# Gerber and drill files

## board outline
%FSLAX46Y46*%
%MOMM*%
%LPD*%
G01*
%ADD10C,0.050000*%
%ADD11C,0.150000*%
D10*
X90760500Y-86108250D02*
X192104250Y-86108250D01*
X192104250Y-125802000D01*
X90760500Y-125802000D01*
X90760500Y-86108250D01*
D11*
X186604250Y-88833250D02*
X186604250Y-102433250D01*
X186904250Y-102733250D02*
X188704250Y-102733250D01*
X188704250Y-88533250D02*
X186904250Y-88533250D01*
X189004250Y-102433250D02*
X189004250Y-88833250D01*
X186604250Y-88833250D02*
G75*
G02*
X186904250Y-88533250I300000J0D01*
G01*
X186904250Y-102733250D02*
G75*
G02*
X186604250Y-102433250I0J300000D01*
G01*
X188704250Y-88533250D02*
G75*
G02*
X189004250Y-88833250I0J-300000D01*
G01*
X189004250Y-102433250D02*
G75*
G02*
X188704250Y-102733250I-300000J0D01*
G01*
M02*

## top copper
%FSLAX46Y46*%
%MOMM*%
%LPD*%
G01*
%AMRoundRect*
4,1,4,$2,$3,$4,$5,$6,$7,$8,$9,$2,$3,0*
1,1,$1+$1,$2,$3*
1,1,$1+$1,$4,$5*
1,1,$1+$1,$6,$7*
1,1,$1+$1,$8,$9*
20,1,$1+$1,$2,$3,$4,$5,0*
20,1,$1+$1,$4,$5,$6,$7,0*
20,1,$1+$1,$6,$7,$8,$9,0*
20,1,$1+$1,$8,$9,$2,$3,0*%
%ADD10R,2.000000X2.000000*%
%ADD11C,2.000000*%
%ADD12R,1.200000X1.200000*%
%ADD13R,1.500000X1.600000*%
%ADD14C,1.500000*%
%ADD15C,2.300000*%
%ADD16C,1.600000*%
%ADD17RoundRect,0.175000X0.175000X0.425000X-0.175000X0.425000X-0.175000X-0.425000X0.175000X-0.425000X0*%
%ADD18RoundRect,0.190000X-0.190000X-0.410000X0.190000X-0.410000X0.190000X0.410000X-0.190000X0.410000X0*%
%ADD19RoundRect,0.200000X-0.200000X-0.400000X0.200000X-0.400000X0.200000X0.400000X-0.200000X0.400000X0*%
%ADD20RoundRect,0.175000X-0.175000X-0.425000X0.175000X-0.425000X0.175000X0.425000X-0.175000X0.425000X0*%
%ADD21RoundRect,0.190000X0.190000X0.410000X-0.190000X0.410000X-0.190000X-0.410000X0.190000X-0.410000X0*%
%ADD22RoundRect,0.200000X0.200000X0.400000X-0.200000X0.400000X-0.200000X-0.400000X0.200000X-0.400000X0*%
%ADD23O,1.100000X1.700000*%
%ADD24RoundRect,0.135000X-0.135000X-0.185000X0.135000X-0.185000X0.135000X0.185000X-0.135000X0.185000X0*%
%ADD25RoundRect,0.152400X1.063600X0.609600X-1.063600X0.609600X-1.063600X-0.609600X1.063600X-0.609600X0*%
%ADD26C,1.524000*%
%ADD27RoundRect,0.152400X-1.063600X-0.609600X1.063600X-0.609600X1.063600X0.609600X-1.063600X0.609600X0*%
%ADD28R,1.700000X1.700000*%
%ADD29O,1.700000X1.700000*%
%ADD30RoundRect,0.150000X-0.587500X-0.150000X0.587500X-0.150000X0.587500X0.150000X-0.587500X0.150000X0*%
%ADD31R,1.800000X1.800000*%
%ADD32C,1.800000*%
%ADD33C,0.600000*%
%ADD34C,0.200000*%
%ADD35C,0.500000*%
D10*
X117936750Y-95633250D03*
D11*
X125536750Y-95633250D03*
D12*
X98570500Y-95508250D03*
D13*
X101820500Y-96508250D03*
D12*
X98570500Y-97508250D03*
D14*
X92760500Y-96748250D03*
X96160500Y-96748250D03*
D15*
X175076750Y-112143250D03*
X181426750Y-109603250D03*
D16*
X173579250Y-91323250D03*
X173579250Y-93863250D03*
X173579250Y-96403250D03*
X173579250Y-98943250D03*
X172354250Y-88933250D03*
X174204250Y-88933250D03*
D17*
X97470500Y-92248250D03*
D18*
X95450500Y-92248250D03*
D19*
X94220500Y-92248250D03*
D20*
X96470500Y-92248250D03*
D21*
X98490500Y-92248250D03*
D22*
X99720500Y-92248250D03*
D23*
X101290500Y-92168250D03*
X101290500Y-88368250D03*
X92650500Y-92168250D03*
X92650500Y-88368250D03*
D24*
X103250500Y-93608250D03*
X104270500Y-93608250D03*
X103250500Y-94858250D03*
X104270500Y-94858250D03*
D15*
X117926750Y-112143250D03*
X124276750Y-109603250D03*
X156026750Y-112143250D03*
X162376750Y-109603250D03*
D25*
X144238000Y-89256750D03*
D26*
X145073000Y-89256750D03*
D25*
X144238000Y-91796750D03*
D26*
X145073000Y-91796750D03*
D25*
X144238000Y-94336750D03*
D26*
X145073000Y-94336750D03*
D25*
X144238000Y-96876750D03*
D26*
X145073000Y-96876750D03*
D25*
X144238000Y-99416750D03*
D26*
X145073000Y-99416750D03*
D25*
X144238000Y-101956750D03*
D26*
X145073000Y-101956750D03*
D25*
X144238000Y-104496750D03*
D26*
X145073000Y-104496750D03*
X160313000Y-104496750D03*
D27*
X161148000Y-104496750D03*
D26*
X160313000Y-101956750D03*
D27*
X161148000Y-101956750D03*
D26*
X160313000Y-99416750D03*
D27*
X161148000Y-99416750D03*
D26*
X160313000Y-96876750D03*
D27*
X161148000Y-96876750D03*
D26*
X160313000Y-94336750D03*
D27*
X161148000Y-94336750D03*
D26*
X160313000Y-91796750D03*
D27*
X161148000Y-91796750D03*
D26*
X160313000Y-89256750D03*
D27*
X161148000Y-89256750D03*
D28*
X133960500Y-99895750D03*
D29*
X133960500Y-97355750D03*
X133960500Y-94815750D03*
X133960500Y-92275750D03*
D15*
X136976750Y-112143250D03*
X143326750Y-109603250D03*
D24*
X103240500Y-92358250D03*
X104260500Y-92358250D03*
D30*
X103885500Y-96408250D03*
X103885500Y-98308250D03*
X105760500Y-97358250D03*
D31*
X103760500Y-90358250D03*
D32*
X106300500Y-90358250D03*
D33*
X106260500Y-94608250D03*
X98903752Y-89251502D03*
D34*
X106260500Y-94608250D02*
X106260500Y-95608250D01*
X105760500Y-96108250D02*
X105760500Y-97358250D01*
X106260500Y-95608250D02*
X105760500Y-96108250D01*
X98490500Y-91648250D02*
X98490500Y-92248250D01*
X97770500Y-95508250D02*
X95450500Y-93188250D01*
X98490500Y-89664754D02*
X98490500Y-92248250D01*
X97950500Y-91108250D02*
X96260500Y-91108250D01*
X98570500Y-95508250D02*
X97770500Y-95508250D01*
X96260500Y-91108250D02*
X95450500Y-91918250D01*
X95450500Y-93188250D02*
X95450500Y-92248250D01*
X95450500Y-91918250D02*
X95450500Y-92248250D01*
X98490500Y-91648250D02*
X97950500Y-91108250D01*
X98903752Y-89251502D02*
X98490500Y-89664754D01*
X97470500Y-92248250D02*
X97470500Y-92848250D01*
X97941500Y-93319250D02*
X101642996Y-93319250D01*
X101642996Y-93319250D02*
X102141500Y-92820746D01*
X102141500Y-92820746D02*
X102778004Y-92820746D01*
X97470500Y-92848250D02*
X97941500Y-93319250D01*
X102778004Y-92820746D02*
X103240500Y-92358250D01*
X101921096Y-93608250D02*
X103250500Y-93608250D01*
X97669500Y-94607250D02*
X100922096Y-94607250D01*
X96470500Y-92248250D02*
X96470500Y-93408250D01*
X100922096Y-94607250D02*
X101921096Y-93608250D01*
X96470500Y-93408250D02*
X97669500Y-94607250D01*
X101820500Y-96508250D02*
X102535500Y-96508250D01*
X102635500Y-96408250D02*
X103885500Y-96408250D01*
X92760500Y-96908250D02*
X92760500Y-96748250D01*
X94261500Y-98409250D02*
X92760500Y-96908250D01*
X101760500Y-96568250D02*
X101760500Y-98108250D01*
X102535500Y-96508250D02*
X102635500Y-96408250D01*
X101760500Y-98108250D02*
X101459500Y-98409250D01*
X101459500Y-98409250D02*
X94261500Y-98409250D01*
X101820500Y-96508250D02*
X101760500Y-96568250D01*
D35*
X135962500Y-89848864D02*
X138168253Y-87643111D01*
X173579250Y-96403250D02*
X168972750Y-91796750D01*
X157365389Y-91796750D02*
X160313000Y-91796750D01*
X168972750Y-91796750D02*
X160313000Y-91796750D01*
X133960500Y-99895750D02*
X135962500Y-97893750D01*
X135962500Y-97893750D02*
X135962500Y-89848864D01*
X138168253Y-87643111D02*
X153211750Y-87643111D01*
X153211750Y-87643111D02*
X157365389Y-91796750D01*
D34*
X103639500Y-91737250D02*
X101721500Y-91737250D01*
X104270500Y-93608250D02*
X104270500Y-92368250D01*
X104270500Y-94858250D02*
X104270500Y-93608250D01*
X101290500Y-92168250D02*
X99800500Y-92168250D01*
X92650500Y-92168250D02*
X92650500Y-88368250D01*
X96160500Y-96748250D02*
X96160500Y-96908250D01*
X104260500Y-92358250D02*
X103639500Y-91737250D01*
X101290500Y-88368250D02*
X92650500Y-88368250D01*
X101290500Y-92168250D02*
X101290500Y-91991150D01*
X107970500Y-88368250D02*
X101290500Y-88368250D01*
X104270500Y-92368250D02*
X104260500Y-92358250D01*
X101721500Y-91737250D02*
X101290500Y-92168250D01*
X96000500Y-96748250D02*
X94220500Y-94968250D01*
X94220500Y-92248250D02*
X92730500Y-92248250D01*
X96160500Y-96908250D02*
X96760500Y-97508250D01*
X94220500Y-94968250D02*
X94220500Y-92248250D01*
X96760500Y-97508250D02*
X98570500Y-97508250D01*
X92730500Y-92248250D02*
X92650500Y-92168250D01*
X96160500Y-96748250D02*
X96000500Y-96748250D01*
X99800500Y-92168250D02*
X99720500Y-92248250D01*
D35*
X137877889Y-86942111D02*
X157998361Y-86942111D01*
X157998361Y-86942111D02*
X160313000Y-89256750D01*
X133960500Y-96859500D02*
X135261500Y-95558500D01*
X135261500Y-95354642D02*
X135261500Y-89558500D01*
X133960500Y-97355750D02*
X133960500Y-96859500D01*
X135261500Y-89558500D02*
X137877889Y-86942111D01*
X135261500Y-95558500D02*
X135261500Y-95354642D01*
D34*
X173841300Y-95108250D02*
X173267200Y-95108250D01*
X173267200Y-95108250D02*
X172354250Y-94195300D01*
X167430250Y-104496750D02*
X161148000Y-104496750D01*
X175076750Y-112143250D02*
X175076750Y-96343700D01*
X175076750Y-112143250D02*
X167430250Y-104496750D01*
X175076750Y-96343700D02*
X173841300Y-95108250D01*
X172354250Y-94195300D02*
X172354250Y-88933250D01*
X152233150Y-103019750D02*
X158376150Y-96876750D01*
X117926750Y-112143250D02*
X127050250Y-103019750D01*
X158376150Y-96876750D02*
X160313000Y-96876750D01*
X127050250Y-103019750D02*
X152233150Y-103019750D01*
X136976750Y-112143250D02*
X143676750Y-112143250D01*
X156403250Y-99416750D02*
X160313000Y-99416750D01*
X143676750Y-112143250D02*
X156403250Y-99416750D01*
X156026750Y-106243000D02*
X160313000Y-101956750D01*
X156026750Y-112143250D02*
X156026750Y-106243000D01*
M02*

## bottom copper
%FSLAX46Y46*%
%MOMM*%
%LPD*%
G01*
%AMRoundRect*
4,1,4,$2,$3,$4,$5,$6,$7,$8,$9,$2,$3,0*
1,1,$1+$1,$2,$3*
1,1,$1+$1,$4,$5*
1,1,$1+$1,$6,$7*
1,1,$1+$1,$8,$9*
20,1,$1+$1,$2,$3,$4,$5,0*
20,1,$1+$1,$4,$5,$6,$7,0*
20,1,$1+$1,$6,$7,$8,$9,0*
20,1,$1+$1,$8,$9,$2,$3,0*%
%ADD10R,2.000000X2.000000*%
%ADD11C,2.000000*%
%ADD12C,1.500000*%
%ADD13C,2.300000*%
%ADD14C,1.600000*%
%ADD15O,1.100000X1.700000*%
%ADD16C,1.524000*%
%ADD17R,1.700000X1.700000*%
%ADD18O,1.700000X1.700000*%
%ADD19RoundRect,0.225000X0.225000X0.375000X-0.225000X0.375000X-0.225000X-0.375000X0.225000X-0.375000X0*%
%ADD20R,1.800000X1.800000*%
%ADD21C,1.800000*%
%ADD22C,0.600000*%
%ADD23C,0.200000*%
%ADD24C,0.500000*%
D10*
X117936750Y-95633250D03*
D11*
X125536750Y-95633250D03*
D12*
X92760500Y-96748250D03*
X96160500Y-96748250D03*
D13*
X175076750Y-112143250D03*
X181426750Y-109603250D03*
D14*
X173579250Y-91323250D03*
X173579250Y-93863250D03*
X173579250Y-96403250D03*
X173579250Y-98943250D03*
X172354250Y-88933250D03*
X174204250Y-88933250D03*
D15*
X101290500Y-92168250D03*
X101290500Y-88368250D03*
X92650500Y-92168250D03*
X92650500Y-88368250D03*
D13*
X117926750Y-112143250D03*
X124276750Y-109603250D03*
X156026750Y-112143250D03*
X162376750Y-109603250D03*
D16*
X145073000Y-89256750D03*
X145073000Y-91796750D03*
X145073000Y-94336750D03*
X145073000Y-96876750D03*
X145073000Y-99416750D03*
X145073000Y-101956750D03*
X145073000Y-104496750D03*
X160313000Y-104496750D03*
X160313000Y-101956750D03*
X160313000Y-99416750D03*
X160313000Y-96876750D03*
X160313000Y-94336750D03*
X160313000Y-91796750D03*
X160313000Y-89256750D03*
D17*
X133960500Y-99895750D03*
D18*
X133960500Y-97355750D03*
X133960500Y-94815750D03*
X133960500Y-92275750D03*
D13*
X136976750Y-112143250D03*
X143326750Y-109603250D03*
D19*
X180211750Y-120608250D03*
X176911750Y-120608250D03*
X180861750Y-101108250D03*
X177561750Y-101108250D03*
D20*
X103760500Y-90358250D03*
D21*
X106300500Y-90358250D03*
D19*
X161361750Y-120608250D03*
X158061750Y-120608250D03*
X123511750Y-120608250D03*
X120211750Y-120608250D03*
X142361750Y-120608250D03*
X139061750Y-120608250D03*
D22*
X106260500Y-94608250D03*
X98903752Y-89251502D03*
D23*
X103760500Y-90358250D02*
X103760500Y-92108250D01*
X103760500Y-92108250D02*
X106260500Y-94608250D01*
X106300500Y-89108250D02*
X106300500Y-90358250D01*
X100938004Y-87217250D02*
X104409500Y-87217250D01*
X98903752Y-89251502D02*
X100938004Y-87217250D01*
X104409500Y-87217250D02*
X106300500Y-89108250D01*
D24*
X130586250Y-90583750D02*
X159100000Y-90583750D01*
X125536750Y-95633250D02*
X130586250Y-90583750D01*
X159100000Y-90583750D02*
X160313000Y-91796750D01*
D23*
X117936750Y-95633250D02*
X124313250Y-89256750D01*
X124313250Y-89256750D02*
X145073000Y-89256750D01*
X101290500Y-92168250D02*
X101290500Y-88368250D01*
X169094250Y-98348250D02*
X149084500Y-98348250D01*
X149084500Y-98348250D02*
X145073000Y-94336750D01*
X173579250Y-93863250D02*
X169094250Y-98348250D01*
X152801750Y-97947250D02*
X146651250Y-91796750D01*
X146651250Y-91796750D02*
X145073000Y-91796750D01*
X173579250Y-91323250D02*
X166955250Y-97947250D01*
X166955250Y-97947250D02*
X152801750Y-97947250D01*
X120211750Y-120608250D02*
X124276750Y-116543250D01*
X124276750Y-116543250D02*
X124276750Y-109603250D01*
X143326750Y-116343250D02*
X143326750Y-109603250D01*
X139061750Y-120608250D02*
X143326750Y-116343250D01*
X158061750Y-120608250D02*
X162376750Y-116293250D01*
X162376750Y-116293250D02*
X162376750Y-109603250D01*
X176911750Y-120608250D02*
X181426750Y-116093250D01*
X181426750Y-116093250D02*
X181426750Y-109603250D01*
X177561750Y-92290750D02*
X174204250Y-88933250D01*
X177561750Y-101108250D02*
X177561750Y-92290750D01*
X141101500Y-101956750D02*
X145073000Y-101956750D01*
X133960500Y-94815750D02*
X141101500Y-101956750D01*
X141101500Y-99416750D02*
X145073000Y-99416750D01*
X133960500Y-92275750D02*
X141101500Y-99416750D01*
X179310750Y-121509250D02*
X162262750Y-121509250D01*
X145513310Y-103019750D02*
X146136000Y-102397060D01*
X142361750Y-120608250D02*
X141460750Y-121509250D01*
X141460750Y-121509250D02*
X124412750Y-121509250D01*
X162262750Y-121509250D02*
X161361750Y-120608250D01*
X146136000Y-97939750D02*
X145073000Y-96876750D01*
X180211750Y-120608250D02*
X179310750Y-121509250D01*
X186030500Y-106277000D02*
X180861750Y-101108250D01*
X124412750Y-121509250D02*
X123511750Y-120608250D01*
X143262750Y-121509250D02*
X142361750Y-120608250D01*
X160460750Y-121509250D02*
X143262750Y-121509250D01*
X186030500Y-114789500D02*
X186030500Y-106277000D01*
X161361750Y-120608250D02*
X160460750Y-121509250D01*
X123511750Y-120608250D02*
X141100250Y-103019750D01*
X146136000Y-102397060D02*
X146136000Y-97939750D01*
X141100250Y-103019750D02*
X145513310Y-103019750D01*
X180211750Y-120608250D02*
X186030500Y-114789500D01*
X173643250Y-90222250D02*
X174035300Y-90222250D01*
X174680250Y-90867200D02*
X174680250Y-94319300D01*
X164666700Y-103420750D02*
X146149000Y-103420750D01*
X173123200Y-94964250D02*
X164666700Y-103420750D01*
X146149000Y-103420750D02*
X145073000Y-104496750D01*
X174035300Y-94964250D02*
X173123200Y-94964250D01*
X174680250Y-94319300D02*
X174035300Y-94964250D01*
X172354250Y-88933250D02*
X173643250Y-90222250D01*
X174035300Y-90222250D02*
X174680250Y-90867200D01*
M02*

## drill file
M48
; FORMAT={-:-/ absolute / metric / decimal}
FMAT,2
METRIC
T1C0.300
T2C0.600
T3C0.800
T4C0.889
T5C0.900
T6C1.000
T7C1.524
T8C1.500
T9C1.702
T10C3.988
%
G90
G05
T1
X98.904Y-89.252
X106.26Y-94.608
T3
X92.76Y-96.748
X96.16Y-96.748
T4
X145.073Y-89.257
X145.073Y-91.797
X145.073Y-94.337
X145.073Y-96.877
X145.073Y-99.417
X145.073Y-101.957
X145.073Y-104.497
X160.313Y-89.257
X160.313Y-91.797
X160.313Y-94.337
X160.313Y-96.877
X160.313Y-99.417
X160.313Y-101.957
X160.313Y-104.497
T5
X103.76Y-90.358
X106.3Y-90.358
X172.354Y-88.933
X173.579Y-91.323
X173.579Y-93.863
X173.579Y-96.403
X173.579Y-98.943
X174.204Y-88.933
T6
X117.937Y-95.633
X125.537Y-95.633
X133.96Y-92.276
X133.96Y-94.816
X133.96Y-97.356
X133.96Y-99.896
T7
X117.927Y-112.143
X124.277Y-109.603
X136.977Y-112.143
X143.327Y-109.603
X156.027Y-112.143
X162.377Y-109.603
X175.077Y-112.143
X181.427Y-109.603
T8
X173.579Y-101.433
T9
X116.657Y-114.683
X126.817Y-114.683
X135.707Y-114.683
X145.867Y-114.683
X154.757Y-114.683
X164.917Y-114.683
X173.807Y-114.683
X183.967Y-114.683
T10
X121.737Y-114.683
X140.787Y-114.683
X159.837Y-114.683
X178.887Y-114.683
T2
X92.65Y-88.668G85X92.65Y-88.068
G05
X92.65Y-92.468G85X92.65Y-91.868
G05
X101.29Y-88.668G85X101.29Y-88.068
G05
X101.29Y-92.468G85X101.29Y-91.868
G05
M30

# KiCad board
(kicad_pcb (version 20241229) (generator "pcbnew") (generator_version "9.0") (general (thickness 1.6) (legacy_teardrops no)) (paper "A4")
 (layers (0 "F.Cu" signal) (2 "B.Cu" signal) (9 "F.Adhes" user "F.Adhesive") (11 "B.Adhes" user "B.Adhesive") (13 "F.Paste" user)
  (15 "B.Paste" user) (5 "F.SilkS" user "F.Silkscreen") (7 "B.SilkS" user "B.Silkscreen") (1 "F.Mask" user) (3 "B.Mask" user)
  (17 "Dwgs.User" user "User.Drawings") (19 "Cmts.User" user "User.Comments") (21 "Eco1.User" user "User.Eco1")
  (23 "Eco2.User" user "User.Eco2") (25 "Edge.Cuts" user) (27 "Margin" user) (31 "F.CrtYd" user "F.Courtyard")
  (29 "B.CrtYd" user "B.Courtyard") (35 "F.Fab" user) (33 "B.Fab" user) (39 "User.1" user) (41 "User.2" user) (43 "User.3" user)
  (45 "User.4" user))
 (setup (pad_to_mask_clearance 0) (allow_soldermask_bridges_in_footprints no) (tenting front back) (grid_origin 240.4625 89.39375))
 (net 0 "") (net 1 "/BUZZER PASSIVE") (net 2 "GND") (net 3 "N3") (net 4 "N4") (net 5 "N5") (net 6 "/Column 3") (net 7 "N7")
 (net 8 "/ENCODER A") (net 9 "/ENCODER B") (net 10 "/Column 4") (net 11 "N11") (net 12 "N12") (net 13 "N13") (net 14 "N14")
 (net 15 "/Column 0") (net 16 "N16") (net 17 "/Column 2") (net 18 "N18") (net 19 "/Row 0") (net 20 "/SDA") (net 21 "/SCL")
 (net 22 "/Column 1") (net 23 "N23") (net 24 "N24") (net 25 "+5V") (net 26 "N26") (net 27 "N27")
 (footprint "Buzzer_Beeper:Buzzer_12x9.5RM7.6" (layer "F.Cu") (at 117.93675 95.63325)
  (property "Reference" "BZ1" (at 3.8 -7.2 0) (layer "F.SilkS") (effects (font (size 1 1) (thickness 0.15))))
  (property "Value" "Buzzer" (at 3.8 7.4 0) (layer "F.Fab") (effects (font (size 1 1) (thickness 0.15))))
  (pad "1" thru_hole rect (at 0 0) (size 2 2) (drill 1) (layers "*.Cu" "*.Mask") (remove_unused_layers no) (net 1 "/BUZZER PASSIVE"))
  (pad "2" thru_hole circle (at 7.6 0) (size 2 2) (drill 1) (layers "*.Cu" "*.Mask") (remove_unused_layers no) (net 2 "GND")))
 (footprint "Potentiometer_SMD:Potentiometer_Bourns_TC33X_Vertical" (layer "F.Cu") (at 100.3705 96.50825)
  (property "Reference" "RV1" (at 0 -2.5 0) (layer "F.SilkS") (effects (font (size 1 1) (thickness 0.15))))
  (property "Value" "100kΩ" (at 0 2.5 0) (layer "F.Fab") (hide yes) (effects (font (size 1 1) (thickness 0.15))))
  (pad "1" smd rect (at -1.8 -1) (size 1.2 1.2) (layers "F.Cu" "F.Mask" "F.Paste") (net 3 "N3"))
  (pad "2" smd rect (at 1.45 0) (size 1.5 1.6) (layers "F.Cu" "F.Mask" "F.Paste") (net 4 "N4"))
  (pad "3" smd rect (at -1.8 1) (size 1.2 1.2) (layers "F.Cu" "F.Mask" "F.Paste") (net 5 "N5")))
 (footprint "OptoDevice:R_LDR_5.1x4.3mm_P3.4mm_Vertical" (layer "F.Cu") (at 92.7605 96.74825)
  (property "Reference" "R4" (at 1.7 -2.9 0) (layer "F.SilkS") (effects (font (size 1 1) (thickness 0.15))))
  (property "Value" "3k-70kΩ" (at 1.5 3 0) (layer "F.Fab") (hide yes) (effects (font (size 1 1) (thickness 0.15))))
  (pad "1" thru_hole circle (at 0 0) (size 1.5 1.5) (drill 0.8) (layers "*.Cu" "*.Mask") (remove_unused_layers no) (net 4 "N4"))
  (pad "2" thru_hole circle (at 3.4 0) (size 1.5 1.5) (drill 0.8) (layers "*.Cu" "*.Mask") (remove_unused_layers no) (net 5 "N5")))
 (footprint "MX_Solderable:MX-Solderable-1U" (layer "F.Cu") (at 178.88675 114.68325)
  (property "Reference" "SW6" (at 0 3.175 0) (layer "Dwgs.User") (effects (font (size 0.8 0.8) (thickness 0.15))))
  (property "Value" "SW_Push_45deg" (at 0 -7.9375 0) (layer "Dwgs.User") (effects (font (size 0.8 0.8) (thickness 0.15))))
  (pad "" np_thru_hole circle (at -5.08 0 48.099) (size 1.7018 1.7018) (drill 1.7018) (layers "*.Cu" "*.Mask"))
  (pad "" np_thru_hole circle (at 0 0) (size 3.9878 3.9878) (drill 3.9878) (layers "*.Cu" "*.Mask"))
  (pad "" np_thru_hole circle (at 5.08 0 48.099) (size 1.7018 1.7018) (drill 1.7018) (layers "*.Cu" "*.Mask"))
  (pad "1" thru_hole circle (at -3.81 -2.54) (size 2.3 2.3) (drill 1.524) (layers "*.Cu" "B.Mask") (remove_unused_layers no)
   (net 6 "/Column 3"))
  (pad "2" thru_hole circle (at 2.54 -5.08) (size 2.3 2.3) (drill 1.524) (layers "*.Cu" "B.Mask") (remove_unused_layers no) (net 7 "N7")))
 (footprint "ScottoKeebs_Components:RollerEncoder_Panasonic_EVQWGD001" (layer "F.Cu") (at 179.20425 95.13325)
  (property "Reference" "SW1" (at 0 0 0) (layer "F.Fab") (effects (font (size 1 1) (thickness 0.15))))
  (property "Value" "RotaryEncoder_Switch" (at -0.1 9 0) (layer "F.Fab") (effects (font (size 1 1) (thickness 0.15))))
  (fp_line (start 7.4 -6.3) (end 7.4 7.3) (stroke (width 0.15) (type solid)) (layer "Edge.Cuts"))
  (fp_line (start 7.7 7.6) (end 9.5 7.6) (stroke (width 0.15) (type solid)) (layer "Edge.Cuts"))
  (fp_line (start 9.5 -6.6) (end 7.7 -6.6) (stroke (width 0.15) (type solid)) (layer "Edge.Cuts"))
  (fp_line (start 9.8 7.3) (end 9.8 -6.3) (stroke (width 0.15) (type solid)) (layer "Edge.Cuts"))
  (fp_arc (start 7.4 -6.3) (mid 7.487868 -6.512132) (end 7.7 -6.6) (stroke (width 0.15) (type solid)) (layer "Edge.Cuts"))
  (fp_arc (start 7.7 7.6) (mid 7.487868 7.512132) (end 7.4 7.3) (stroke (width 0.15) (type solid)) (layer "Edge.Cuts"))
  (fp_arc (start 9.5 -6.6) (mid 9.712132 -6.512132) (end 9.8 -6.3) (stroke (width 0.15) (type solid)) (layer "Edge.Cuts"))
  (fp_arc (start 9.8 7.3) (mid 9.712132 7.512132) (end 9.5 7.6) (stroke (width 0.15) (type solid)) (layer "Edge.Cuts"))
  (pad "" np_thru_hole circle (at -5.625 6.3) (size 1.5 1.5) (drill 1.5) (layers "*.Cu" "*.Mask"))
  (pad "A" thru_hole circle (at -5.625 -3.81) (size 1.6 1.6) (drill 0.9) (layers "*.Cu" "*.Mask") (remove_unused_layers no)
   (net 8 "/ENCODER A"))
  (pad "B" thru_hole circle (at -5.625 -1.27) (size 1.6 1.6) (drill 0.9) (layers "*.Cu" "*.Mask") (remove_unused_layers no)
   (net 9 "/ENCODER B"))
  (pad "C" thru_hole circle (at -5.625 1.27) (size 1.6 1.6) (drill 0.9) (layers "*.Cu" "*.Mask") (remove_unused_layers no) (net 2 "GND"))
  (pad "D" thru_hole circle (at -5.625 3.81) (size 1.6 1.6) (drill 0.9) (layers "*.Cu" "*.Mask") (remove_unused_layers no))
  (pad "S1" thru_hole circle (at -6.85 -6.2) (size 1.6 1.6) (drill 0.9) (layers "*.Cu" "*.Mask") (remove_unused_layers no)
   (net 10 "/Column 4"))
  (pad "S2" thru_hole circle (at -5 -6.2) (size 1.6 1.6) (drill 0.9) (layers "*.Cu" "*.Mask") (remove_unused_layers no) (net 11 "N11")))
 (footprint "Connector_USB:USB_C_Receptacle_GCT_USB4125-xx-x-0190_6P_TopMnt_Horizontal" (layer "F.Cu") (at 96.9705 89.16825 180)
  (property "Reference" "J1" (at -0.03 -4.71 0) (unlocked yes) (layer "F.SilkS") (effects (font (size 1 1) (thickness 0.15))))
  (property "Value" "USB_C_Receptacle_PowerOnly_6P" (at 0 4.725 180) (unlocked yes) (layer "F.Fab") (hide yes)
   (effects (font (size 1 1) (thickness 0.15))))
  (pad "A5" smd roundrect (at -0.5 -3.08 180) (size 0.7 1.2) (layers "F.Cu" "F.Mask" "F.Paste") (roundrect_rratio 0.25) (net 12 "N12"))
  (pad "A9" smd roundrect (at 1.52 -3.08) (size 0.76 1.2) (layers "F.Cu" "F.Mask" "F.Paste") (roundrect_rratio 0.25) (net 3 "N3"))
  (pad "A12" smd roundrect (at 2.75 -3.08) (size 0.8 1.2) (layers "F.Cu" "F.Mask" "F.Paste") (roundrect_rratio 0.25) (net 5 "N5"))
  (pad "B5" smd roundrect (at 0.5 -3.08) (size 0.7 1.2) (layers "F.Cu" "F.Mask" "F.Paste") (roundrect_rratio 0.25) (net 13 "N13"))
  (pad "B9" smd roundrect (at -1.52 -3.08 180) (size 0.76 1.2) (layers "F.Cu" "F.Mask" "F.Paste") (roundrect_rratio 0.25) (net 3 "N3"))
  (pad "B12" smd roundrect (at -2.75 -3.08 180) (size 0.8 1.2) (layers "F.Cu" "F.Mask" "F.Paste") (roundrect_rratio 0.25) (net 5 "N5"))
  (pad "S1" thru_hole oval (at -4.32 -3 180) (size 1.1 1.7) (drill oval 0.6 1.2) (layers "*.Cu" "*.Mask" "F.Paste")
   (remove_unused_layers no) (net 5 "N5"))
  (pad "S1" thru_hole oval (at -4.32 0.8 180) (size 1.1 1.7) (drill oval 0.6 1.2) (layers "*.Cu" "*.Mask" "F.Paste")
   (remove_unused_layers no) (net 5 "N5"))
  (pad "S1" thru_hole oval (at 4.32 -3 180) (size 1.1 1.7) (drill oval 0.6 1.2) (layers "*.Cu" "*.Mask" "F.Paste") (remove_unused_layers no)
   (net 5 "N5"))
  (pad "S1" thru_hole oval (at 4.32 0.8 180) (size 1.1 1.7) (drill oval 0.6 1.2) (layers "*.Cu" "*.Mask" "F.Paste")
   (remove_unused_layers no) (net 5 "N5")))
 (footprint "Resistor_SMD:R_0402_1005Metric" (layer "F.Cu") (at 103.7605 93.60825)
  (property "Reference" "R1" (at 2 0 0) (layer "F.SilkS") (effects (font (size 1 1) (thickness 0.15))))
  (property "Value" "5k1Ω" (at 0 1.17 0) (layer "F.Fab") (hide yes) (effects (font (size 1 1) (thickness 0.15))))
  (pad "1" smd roundrect (at -0.51 0) (size 0.54 0.64) (layers "F.Cu" "F.Mask" "F.Paste") (roundrect_rratio 0.25) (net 13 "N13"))
  (pad "2" smd roundrect (at 0.51 0) (size 0.54 0.64) (layers "F.Cu" "F.Mask" "F.Paste") (roundrect_rratio 0.25) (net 5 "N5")))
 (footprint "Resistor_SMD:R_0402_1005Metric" (layer "F.Cu") (at 103.7605 94.85825)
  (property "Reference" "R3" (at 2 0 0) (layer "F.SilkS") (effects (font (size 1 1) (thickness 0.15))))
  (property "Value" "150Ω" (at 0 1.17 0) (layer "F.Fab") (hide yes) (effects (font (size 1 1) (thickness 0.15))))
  (pad "1" smd roundrect (at -0.51 0) (size 0.54 0.64) (layers "F.Cu" "F.Mask" "F.Paste") (roundrect_rratio 0.25) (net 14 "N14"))
  (pad "2" smd roundrect (at 0.51 0) (size 0.54 0.64) (layers "F.Cu" "F.Mask" "F.Paste") (roundrect_rratio 0.25) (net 5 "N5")))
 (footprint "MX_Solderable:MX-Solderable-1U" (layer "F.Cu") (at 121.73675 114.68325)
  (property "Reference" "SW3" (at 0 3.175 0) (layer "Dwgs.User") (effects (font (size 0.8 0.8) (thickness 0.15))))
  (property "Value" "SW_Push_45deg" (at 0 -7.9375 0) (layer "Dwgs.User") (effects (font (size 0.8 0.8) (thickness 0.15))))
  (pad "" np_thru_hole circle (at -5.08 0 48.099) (size 1.7018 1.7018) (drill 1.7018) (layers "*.Cu" "*.Mask"))
  (pad "" np_thru_hole circle (at 0 0) (size 3.9878 3.9878) (drill 3.9878) (layers "*.Cu" "*.Mask"))
  (pad "" np_thru_hole circle (at 5.08 0 48.099) (size 1.7018 1.7018) (drill 1.7018) (layers "*.Cu" "*.Mask"))
  (pad "1" thru_hole circle (at -3.81 -2.54) (size 2.3 2.3) (drill 1.524) (layers "*.Cu" "B.Mask") (remove_unused_layers no)
   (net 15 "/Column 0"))
  (pad "2" thru_hole circle (at 2.54 -5.08) (size 2.3 2.3) (drill 1.524) (layers "*.Cu" "B.Mask") (remove_unused_layers no) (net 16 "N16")))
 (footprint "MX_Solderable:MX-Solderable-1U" (layer "F.Cu") (at 159.83675 114.68325)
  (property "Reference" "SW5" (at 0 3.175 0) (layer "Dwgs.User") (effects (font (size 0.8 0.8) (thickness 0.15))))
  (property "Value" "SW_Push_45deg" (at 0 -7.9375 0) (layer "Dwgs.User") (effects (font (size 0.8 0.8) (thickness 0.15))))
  (pad "" np_thru_hole circle (at -5.08 0 48.099) (size 1.7018 1.7018) (drill 1.7018) (layers "*.Cu" "*.Mask"))
  (pad "" np_thru_hole circle (at 0 0) (size 3.9878 3.9878) (drill 3.9878) (layers "*.Cu" "*.Mask"))
  (pad "" np_thru_hole circle (at 5.08 0 48.099) (size 1.7018 1.7018) (drill 1.7018) (layers "*.Cu" "*.Mask"))
  (pad "1" thru_hole circle (at -3.81 -2.54) (size 2.3 2.3) (drill 1.524) (layers "*.Cu" "B.Mask") (remove_unused_layers no)
   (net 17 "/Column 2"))
  (pad "2" thru_hole circle (at 2.54 -5.08) (size 2.3 2.3) (drill 1.524) (layers "*.Cu" "B.Mask") (remove_unused_layers no) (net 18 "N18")))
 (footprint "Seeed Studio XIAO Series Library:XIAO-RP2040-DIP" (layer "F.Cu") (at 152.693 96.87675)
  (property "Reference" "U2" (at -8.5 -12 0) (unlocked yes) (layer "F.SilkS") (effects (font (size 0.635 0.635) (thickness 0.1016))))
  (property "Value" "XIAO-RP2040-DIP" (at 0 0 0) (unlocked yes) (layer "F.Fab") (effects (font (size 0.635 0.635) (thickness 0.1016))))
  (pad "1" smd roundrect (at -8.455 -7.62 180) (size 2.432 1.524) (layers "F.Cu" "F.Mask") (roundrect_rratio 0.1) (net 1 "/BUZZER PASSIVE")
   (thermal_bridge_angle 45))
  (pad "1" thru_hole circle (at -7.62 -7.62 180) (size 1.524 1.524) (drill 0.889) (layers "*.Cu" "*.Mask") (remove_unused_layers no)
   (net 1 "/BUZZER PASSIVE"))
  (pad "2" smd roundrect (at -8.455 -5.08 180) (size 2.432 1.524) (layers "F.Cu" "F.Mask") (roundrect_rratio 0.1) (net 8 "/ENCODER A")
   (thermal_bridge_angle 45))
  (pad "2" thru_hole circle (at -7.62 -5.08 180) (size 1.524 1.524) (drill 0.889) (layers "*.Cu" "*.Mask") (remove_unused_layers no)
   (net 8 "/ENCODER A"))
  (pad "3" smd roundrect (at -8.455 -2.54 180) (size 2.432 1.524) (layers "F.Cu" "F.Mask") (roundrect_rratio 0.1) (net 9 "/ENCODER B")
   (thermal_bridge_angle 45))
  (pad "3" thru_hole circle (at -7.62 -2.54 180) (size 1.524 1.524) (drill 0.889) (layers "*.Cu" "*.Mask") (remove_unused_layers no)
   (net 9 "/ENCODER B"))
  (pad "4" smd roundrect (at -8.455 0 180) (size 2.432 1.524) (layers "F.Cu" "F.Mask") (roundrect_rratio 0.1) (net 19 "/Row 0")
   (thermal_bridge_angle 45))
  (pad "4" thru_hole circle (at -7.62 0 180) (size 1.524 1.524) (drill 0.889) (layers "*.Cu" "*.Mask") (remove_unused_layers no)
   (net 19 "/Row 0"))
  (pad "5" smd roundrect (at -8.455 2.54 180) (size 2.432 1.524) (layers "F.Cu" "F.Mask") (roundrect_rratio 0.1) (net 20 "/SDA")
   (thermal_bridge_angle 45))
  (pad "5" thru_hole circle (at -7.62 2.54 180) (size 1.524 1.524) (drill 0.889) (layers "*.Cu" "*.Mask") (remove_unused_layers no)
   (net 20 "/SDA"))
  (pad "6" smd roundrect (at -8.455 5.08 180) (size 2.432 1.524) (layers "F.Cu" "F.Mask") (roundrect_rratio 0.1) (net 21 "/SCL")
   (thermal_bridge_angle 45))
  (pad "6" thru_hole circle (at -7.62 5.08 180) (size 1.524 1.524) (drill 0.889) (layers "*.Cu" "*.Mask") (remove_unused_layers no)
   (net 21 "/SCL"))
  (pad "7" smd roundrect (at -8.455 7.62 180) (size 2.432 1.524) (layers "F.Cu" "F.Mask") (roundrect_rratio 0.1) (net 10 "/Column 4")
   (thermal_bridge_angle 45))
  (pad "7" thru_hole circle (at -7.62 7.62 180) (size 1.524 1.524) (drill 0.889) (layers "*.Cu" "*.Mask") (remove_unused_layers no)
   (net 10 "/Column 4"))
  (pad "8" thru_hole circle (at 7.62 7.62) (size 1.524 1.524) (drill 0.889) (layers "*.Cu" "*.Mask") (remove_unused_layers no)
   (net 6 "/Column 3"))
  (pad "8" smd roundrect (at 8.455 7.62) (size 2.432 1.524) (layers "F.Cu" "F.Mask") (roundrect_rratio 0.1) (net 6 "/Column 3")
   (thermal_bridge_angle 45))
  (pad "9" thru_hole circle (at 7.62 5.08) (size 1.524 1.524) (drill 0.889) (layers "*.Cu" "*.Mask") (remove_unused_layers no)
   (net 17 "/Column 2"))
  (pad "9" smd roundrect (at 8.455 5.08) (size 2.432 1.524) (layers "F.Cu" "F.Mask") (roundrect_rratio 0.1) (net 17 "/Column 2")
   (thermal_bridge_angle 45))
  (pad "10" thru_hole circle (at 7.62 2.54) (size 1.524 1.524) (drill 0.889) (layers "*.Cu" "*.Mask") (remove_unused_layers no)
   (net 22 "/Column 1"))
  (pad "10" smd roundrect (at 8.455 2.54) (size 2.432 1.524) (layers "F.Cu" "F.Mask") (roundrect_rratio 0.1) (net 22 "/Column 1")
   (thermal_bridge_angle 45))
  (pad "11" thru_hole circle (at 7.62 0) (size 1.524 1.524) (drill 0.889) (layers "*.Cu" "*.Mask") (remove_unused_layers no)
   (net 15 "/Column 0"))
  (pad "11" smd roundrect (at 8.455 0) (size 2.432 1.524) (layers "F.Cu" "F.Mask") (roundrect_rratio 0.1) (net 15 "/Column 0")
   (thermal_bridge_angle 45))
  (pad "12" thru_hole circle (at 7.62 -2.54) (size 1.524 1.524) (drill 0.889) (layers "*.Cu" "*.Mask") (remove_unused_layers no)
   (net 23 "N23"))
  (pad "12" smd roundrect (at 8.455 -2.54) (size 2.432 1.524) (layers "F.Cu" "F.Mask") (roundrect_rratio 0.1) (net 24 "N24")
   (thermal_bridge_angle 45))
  (pad "13" thru_hole circle (at 7.62 -5.08) (size 1.524 1.524) (drill 0.889) (layers "*.Cu" "*.Mask") (remove_unused_layers no)
   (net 2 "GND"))
  (pad "13" smd roundrect (at 8.455 -5.08) (size 2.432 1.524) (layers "F.Cu" "F.Mask") (roundrect_rratio 0.1) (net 2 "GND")
   (thermal_bridge_angle 45))
  (pad "14" thru_hole circle (at 7.62 -7.62) (size 1.524 1.524) (drill 0.889) (layers "*.Cu" "*.Mask") (remove_unused_layers no)
   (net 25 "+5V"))
  (pad "14" smd roundrect (at 8.455 -7.62) (size 2.432 1.524) (layers "F.Cu" "F.Mask") (roundrect_rratio 0.1) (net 25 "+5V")
   (thermal_bridge_angle 45)))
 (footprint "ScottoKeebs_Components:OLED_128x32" (layer "F.Cu") (at 132.3605 90.09575)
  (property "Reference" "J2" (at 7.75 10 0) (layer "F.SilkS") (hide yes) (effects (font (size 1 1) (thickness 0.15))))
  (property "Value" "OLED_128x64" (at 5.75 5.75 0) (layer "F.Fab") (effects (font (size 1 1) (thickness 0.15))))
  (pad "1" thru_hole rect (at 1.6 9.8 180) (size 1.7 1.7) (drill 1) (layers "*.Cu" "*.Mask") (remove_unused_layers no) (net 2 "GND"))
  (pad "2" thru_hole oval (at 1.6 7.26 180) (size 1.7 1.7) (drill 1) (layers "*.Cu" "*.Mask") (remove_unused_layers no) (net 25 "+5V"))
  (pad "3" thru_hole oval (at 1.6 4.72 180) (size 1.7 1.7) (drill 1) (layers "*.Cu" "*.Mask") (remove_unused_layers no) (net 21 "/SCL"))
  (pad "4" thru_hole oval (at 1.6 2.18 180) (size 1.7 1.7) (drill 1) (layers "*.Cu" "*.Mask") (remove_unused_layers no) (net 20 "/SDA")))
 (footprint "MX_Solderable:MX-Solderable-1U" (layer "F.Cu") (at 140.78675 114.68325)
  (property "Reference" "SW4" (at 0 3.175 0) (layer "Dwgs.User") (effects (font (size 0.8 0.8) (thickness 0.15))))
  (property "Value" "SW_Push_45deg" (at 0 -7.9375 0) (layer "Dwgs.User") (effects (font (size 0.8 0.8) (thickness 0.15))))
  (pad "" np_thru_hole circle (at -5.08 0 48.099) (size 1.7018 1.7018) (drill 1.7018) (layers "*.Cu" "*.Mask"))
  (pad "" np_thru_hole circle (at 0 0) (size 3.9878 3.9878) (drill 3.9878) (layers "*.Cu" "*.Mask"))
  (pad "" np_thru_hole circle (at 5.08 0 48.099) (size 1.7018 1.7018) (drill 1.7018) (layers "*.Cu" "*.Mask"))
  (pad "1" thru_hole circle (at -3.81 -2.54) (size 2.3 2.3) (drill 1.524) (layers "*.Cu" "B.Mask") (remove_unused_layers no)
   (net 22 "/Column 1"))
  (pad "2" thru_hole circle (at 2.54 -5.08) (size 2.3 2.3) (drill 1.524) (layers "*.Cu" "B.Mask") (remove_unused_layers no) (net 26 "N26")))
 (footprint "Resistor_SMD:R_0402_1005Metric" (layer "F.Cu") (at 103.7505 92.35825)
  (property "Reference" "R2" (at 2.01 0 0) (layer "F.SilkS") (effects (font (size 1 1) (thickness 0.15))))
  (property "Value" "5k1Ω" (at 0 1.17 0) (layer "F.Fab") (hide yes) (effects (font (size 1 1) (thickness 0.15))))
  (pad "1" smd roundrect (at -0.51 0) (size 0.54 0.64) (layers "F.Cu" "F.Mask" "F.Paste") (roundrect_rratio 0.25) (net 12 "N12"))
  (pad "2" smd roundrect (at 0.51 0) (size 0.54 0.64) (layers "F.Cu" "F.Mask" "F.Paste") (roundrect_rratio 0.25) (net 5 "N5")))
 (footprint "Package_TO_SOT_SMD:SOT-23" (layer "F.Cu") (at 104.823 97.35825)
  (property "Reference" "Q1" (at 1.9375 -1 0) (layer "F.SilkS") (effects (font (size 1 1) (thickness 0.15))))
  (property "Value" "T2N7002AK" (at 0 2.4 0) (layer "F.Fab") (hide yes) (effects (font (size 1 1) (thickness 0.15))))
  (pad "1" smd roundrect (at -0.9375 -0.95) (size 1.475 0.6) (layers "F.Cu" "F.Mask" "F.Paste") (roundrect_rratio 0.25) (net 4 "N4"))
  (pad "2" smd roundrect (at -0.9375 0.95) (size 1.475 0.6) (layers "F.Cu" "F.Mask" "F.Paste") (roundrect_rratio 0.25) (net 14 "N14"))
  (pad "3" smd roundrect (at 0.9375 0) (size 1.475 0.6) (layers "F.Cu" "F.Mask" "F.Paste") (roundrect_rratio 0.25) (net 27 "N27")))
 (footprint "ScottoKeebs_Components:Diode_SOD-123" (layer "B.Cu") (at 178.56175 120.60825 180)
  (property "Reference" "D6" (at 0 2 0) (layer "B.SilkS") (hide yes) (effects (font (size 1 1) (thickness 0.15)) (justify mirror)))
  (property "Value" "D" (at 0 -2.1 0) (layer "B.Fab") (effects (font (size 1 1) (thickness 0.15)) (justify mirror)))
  (pad "1" smd roundrect (at -1.65 0 180) (size 0.9 1.2) (layers "B.Cu" "B.Mask" "B.Paste") (roundrect_rratio 0.25) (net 19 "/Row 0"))
  (pad "2" smd roundrect (at 1.65 0 180) (size 0.9 1.2) (layers "B.Cu" "B.Mask" "B.Paste") (roundrect_rratio 0.25) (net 7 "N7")))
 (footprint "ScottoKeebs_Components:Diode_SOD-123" (layer "B.Cu") (at 179.21175 101.10825 180)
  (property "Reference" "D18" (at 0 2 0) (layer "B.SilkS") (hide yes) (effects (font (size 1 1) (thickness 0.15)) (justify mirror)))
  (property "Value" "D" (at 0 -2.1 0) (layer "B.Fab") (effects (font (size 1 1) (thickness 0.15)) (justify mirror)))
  (pad "1" smd roundrect (at -1.65 0 180) (size 0.9 1.2) (layers "B.Cu" "B.Mask" "B.Paste") (roundrect_rratio 0.25) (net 19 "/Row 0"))
  (pad "2" smd roundrect (at 1.65 0 180) (size 0.9 1.2) (layers "B.Cu" "B.Mask" "B.Paste") (roundrect_rratio 0.25) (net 11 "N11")))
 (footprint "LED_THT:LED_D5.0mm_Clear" (layer "B.Cu") (at 103.7605 90.35825)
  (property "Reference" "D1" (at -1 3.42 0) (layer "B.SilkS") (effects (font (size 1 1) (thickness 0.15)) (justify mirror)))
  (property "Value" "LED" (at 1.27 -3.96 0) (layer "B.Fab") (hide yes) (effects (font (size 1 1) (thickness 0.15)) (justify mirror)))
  (pad "1" thru_hole rect (at 0 0) (size 1.8 1.8) (drill 0.9) (layers "*.Cu" "*.Mask") (remove_unused_layers no) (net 27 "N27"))
  (pad "2" thru_hole circle (at 2.54 0) (size 1.8 1.8) (drill 0.9) (layers "*.Cu" "*.Mask") (remove_unused_layers no) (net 3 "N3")))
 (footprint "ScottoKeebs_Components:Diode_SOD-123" (layer "B.Cu") (at 159.71175 120.60825 180)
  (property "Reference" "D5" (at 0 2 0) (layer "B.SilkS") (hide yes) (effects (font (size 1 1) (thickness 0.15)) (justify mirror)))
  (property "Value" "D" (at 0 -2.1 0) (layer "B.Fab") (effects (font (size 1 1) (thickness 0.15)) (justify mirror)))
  (pad "1" smd roundrect (at -1.65 0 180) (size 0.9 1.2) (layers "B.Cu" "B.Mask" "B.Paste") (roundrect_rratio 0.25) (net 19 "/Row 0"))
  (pad "2" smd roundrect (at 1.65 0 180) (size 0.9 1.2) (layers "B.Cu" "B.Mask" "B.Paste") (roundrect_rratio 0.25) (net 18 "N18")))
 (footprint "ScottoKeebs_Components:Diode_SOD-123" (layer "B.Cu") (at 121.86175 120.60825 180)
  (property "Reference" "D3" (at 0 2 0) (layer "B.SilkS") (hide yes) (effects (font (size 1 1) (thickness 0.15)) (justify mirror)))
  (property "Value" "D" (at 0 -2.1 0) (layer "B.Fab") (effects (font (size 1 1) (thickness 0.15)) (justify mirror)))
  (pad "1" smd roundrect (at -1.65 0 180) (size 0.9 1.2) (layers "B.Cu" "B.Mask" "B.Paste") (roundrect_rratio 0.25) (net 19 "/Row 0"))
  (pad "2" smd roundrect (at 1.65 0 180) (size 0.9 1.2) (layers "B.Cu" "B.Mask" "B.Paste") (roundrect_rratio 0.25) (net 16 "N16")))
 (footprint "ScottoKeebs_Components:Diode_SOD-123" (layer "B.Cu") (at 140.71175 120.60825 180)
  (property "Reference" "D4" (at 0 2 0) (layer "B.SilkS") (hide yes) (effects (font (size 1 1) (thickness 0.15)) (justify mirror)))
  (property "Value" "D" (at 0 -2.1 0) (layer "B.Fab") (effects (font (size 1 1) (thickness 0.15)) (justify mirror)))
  (pad "1" smd roundrect (at -1.65 0 180) (size 0.9 1.2) (layers "B.Cu" "B.Mask" "B.Paste") (roundrect_rratio 0.25) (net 19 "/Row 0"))
  (pad "2" smd roundrect (at 1.65 0 180) (size 0.9 1.2) (layers "B.Cu" "B.Mask" "B.Paste") (roundrect_rratio 0.25) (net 26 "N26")))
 (gr_rect (start 90.7605 86.10825) (end 192.10425 125.802) (stroke (width 0.05) (type default)) (fill no) (layer "Edge.Cuts"))
 (segment (start 106.2605 94.60825) (end 106.2605 95.60825) (width 0.2) (layer "F.Cu") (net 27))
 (segment (start 105.7605 96.10825) (end 105.7605 97.35825) (width 0.2) (layer "F.Cu") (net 27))
 (segment (start 106.2605 95.60825) (end 105.7605 96.10825) (width 0.2) (layer "F.Cu") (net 27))
 (via blind (at 106.2605 94.60825) (size 0.6) (drill 0.3) (layers "F.Cu" "B.Cu") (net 27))
 (segment (start 103.7605 90.35825) (end 103.7605 92.10825) (width 0.2) (layer "B.Cu") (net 27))
 (segment (start 103.7605 92.10825) (end 106.2605 94.60825) (width 0.2) (layer "B.Cu") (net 27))
 (segment (start 98.4905 91.64825) (end 98.4905 92.24825) (width 0.2) (layer "F.Cu") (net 3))
 (segment (start 97.7705 95.50825) (end 95.4505 93.18825) (width 0.2) (layer "F.Cu") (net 3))
 (segment (start 98.4905 89.664754) (end 98.4905 92.24825) (width 0.2) (layer "F.Cu") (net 3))
 (segment (start 97.9505 91.10825) (end 96.2605 91.10825) (width 0.2) (layer "F.Cu") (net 3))
 (segment (start 98.5705 95.50825) (end 97.7705 95.50825) (width 0.2) (layer "F.Cu") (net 3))
 (segment (start 96.2605 91.10825) (end 95.4505 91.91825) (width 0.2) (layer "F.Cu") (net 3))
 (segment (start 95.4505 93.18825) (end 95.4505 92.24825) (width 0.2) (layer "F.Cu") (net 3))
 (segment (start 95.4505 91.91825) (end 95.4505 92.24825) (width 0.2) (layer "F.Cu") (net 3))
 (segment (start 98.4905 91.64825) (end 97.9505 91.10825) (width 0.2) (layer "F.Cu") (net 3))
 (segment (start 98.903752 89.251502) (end 98.4905 89.664754) (width 0.2) (layer "F.Cu") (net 3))
 (via blind (at 98.903752 89.251502) (size 0.6) (drill 0.3) (layers "F.Cu" "B.Cu") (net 3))
 (segment (start 106.3005 89.10825) (end 106.3005 90.35825) (width 0.2) (layer "B.Cu") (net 3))
 (segment (start 100.938004 87.21725) (end 104.4095 87.21725) (width 0.2) (layer "B.Cu") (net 3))
 (segment (start 98.903752 89.251502) (end 100.938004 87.21725) (width 0.2) (layer "B.Cu") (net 3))
 (segment (start 104.4095 87.21725) (end 106.3005 89.10825) (width 0.2) (layer "B.Cu") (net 3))
 (segment (start 97.4705 92.24825) (end 97.4705 92.84825) (width 0.2) (layer "F.Cu") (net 12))
 (segment (start 97.9415 93.31925) (end 101.642996 93.31925) (width 0.2) (layer "F.Cu") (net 12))
 (segment (start 101.642996 93.31925) (end 102.1415 92.820746) (width 0.2) (layer "F.Cu") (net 12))
 (segment (start 102.1415 92.820746) (end 102.778004 92.820746) (width 0.2) (layer "F.Cu") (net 12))
 (segment (start 97.4705 92.84825) (end 97.9415 93.31925) (width 0.2) (layer "F.Cu") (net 12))
 (segment (start 102.778004 92.820746) (end 103.2405 92.35825) (width 0.2) (layer "F.Cu") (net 12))
 (segment (start 101.921096 93.60825) (end 103.2505 93.60825) (width 0.2) (layer "F.Cu") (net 13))
 (segment (start 97.6695 94.60725) (end 100.922096 94.60725) (width 0.2) (layer "F.Cu") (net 13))
 (segment (start 96.4705 92.24825) (end 96.4705 93.40825) (width 0.2) (layer "F.Cu") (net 13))
 (segment (start 100.922096 94.60725) (end 101.921096 93.60825) (width 0.2) (layer "F.Cu") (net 13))
 (segment (start 96.4705 93.40825) (end 97.6695 94.60725) (width 0.2) (layer "F.Cu") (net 13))
 (segment (start 101.8205 96.50825) (end 102.5355 96.50825) (width 0.2) (layer "F.Cu") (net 4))
 (segment (start 102.6355 96.40825) (end 103.8855 96.40825) (width 0.2) (layer "F.Cu") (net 4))
 (segment (start 92.7605 96.90825) (end 92.7605 96.74825) (width 0.2) (layer "F.Cu") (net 4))
 (segment (start 94.2615 98.40925) (end 92.7605 96.90825) (width 0.2) (layer "F.Cu") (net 4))
 (segment (start 101.7605 96.56825) (end 101.7605 98.10825) (width 0.2) (layer "F.Cu") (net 4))
 (segment (start 102.5355 96.50825) (end 102.6355 96.40825) (width 0.2) (layer "F.Cu") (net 4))
 (segment (start 101.7605 98.10825) (end 101.4595 98.40925) (width 0.2) (layer "F.Cu") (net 4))
 (segment (start 101.4595 98.40925) (end 94.2615 98.40925) (width 0.2) (layer "F.Cu") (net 4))
 (segment (start 101.8205 96.50825) (end 101.7605 96.56825) (width 0.2) (layer "F.Cu") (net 4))
 (segment (start 135.9625 89.848864) (end 138.168253 87.643111) (width 0.5) (layer "F.Cu") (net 2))
 (segment (start 173.57925 96.40325) (end 168.97275 91.79675) (width 0.5) (layer "F.Cu") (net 2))
 (segment (start 157.365389 91.79675) (end 160.313 91.79675) (width 0.5) (layer "F.Cu") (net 2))
 (segment (start 168.97275 91.79675) (end 160.313 91.79675) (width 0.5) (layer "F.Cu") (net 2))
 (segment (start 133.9605 99.89575) (end 135.9625 97.89375) (width 0.5) (layer "F.Cu") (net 2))
 (segment (start 135.9625 97.89375) (end 135.9625 89.848864) (width 0.5) (layer "F.Cu") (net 2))
 (segment (start 138.168253 87.643111) (end 153.21175 87.643111) (width 0.5) (layer "F.Cu") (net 2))
 (segment (start 153.21175 87.643111) (end 157.365389 91.79675) (width 0.5) (layer "F.Cu") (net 2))
 (segment (start 130.58625 90.58375) (end 159.1 90.58375) (width 0.5) (layer "B.Cu") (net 2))
 (segment (start 125.53675 95.63325) (end 130.58625 90.58375) (width 0.5) (layer "B.Cu") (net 2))
 (segment (start 159.1 90.58375) (end 160.313 91.79675) (width 0.5) (layer "B.Cu") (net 2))
 (segment (start 117.93675 95.63325) (end 124.31325 89.25675) (width 0.2) (layer "B.Cu") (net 1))
 (segment (start 124.31325 89.25675) (end 145.073 89.25675) (width 0.2) (layer "B.Cu") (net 1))
 (segment (start 103.6395 91.73725) (end 101.7215 91.73725) (width 0.2) (layer "F.Cu") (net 5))
 (segment (start 104.2705 93.60825) (end 104.2705 92.36825) (width 0.2) (layer "F.Cu") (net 5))
 (segment (start 104.2705 94.85825) (end 104.2705 93.60825) (width 0.2) (layer "F.Cu") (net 5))
 (segment (start 101.2905 92.16825) (end 99.8005 92.16825) (width 0.2) (layer "F.Cu") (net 5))
 (segment (start 92.6505 92.16825) (end 92.6505 88.36825) (width 0.2) (layer "F.Cu") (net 5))
 (segment (start 96.1605 96.74825) (end 96.1605 96.90825) (width 0.2) (layer "F.Cu") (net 5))
 (segment (start 104.2605 92.35825) (end 103.6395 91.73725) (width 0.2) (layer "F.Cu") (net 5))
 (segment (start 101.2905 88.36825) (end 92.6505 88.36825) (width 0.2) (layer "F.Cu") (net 5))
 (segment (start 101.2905 92.16825) (end 101.2905 91.99115) (width 0.2) (layer "F.Cu") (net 5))
 (segment (start 107.9705 88.36825) (end 101.2905 88.36825) (width 0.2) (layer "F.Cu") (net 5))
 (segment (start 104.2705 92.36825) (end 104.2605 92.35825) (width 0.2) (layer "F.Cu") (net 5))
 (segment (start 101.7215 91.73725) (end 101.2905 92.16825) (width 0.2) (layer "F.Cu") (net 5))
 (segment (start 96.0005 96.74825) (end 94.2205 94.96825) (width 0.2) (layer "F.Cu") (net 5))
 (segment (start 94.2205 92.24825) (end 92.7305 92.24825) (width 0.2) (layer "F.Cu") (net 5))
 (segment (start 96.1605 96.90825) (end 96.7605 97.50825) (width 0.2) (layer "F.Cu") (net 5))
 (segment (start 94.2205 94.96825) (end 94.2205 92.24825) (width 0.2) (layer "F.Cu") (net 5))
 (segment (start 96.7605 97.50825) (end 98.5705 97.50825) (width 0.2) (layer "F.Cu") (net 5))
 (segment (start 92.7305 92.24825) (end 92.6505 92.16825) (width 0.2) (layer "F.Cu") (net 5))
 (segment (start 96.1605 96.74825) (end 96.0005 96.74825) (width 0.2) (layer "F.Cu") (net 5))
 (segment (start 99.8005 92.16825) (end 99.7205 92.24825) (width 0.2) (layer "F.Cu") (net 5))
 (segment (start 101.2905 92.16825) (end 101.2905 88.36825) (width 0.2) (layer "B.Cu") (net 5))
 (segment (start 137.877889 86.942111) (end 157.998361 86.942111) (width 0.5) (layer "F.Cu") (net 25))
 (segment (start 157.998361 86.942111) (end 160.313 89.25675) (width 0.5) (layer "F.Cu") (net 25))
 (segment (start 133.9605 96.8595) (end 135.2615 95.5585) (width 0.5) (layer "F.Cu") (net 25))
 (segment (start 135.2615 95.354642) (end 135.2615 89.5585) (width 0.5) (layer "F.Cu") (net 25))
 (segment (start 133.9605 97.35575) (end 133.9605 96.8595) (width 0.5) (layer "F.Cu") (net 25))
 (segment (start 135.2615 89.5585) (end 137.877889 86.942111) (width 0.5) (layer "F.Cu") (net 25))
 (segment (start 135.2615 95.5585) (end 135.2615 95.354642) (width 0.5) (layer "F.Cu") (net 25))
 (segment (start 169.09425 98.34825) (end 149.0845 98.34825) (width 0.2) (layer "B.Cu") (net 9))
 (segment (start 149.0845 98.34825) (end 145.073 94.33675) (width 0.2) (layer "B.Cu") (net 9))
 (segment (start 173.57925 93.86325) (end 169.09425 98.34825) (width 0.2) (layer "B.Cu") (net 9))
 (segment (start 152.80175 97.94725) (end 146.65125 91.79675) (width 0.2) (layer "B.Cu") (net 8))
 (segment (start 146.65125 91.79675) (end 145.073 91.79675) (width 0.2) (layer "B.Cu") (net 8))
 (segment (start 173.57925 91.32325) (end 166.95525 97.94725) (width 0.2) (layer "B.Cu") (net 8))
 (segment (start 166.95525 97.94725) (end 152.80175 97.94725) (width 0.2) (layer "B.Cu") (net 8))
 (segment (start 120.21175 120.60825) (end 124.27675 116.54325) (width 0.2) (layer "B.Cu") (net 16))
 (segment (start 124.27675 116.54325) (end 124.27675 109.60325) (width 0.2) (layer "B.Cu") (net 16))
 (segment (start 143.32675 116.34325) (end 143.32675 109.60325) (width 0.2) (layer "B.Cu") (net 26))
 (segment (start 139.06175 120.60825) (end 143.32675 116.34325) (width 0.2) (layer "B.Cu") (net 26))
 (segment (start 158.06175 120.60825) (end 162.37675 116.29325) (width 0.2) (layer "B.Cu") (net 18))
 (segment (start 162.37675 116.29325) (end 162.37675 109.60325) (width 0.2) (layer "B.Cu") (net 18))
 (segment (start 176.91175 120.60825) (end 181.42675 116.09325) (width 0.2) (layer "B.Cu") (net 7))
 (segment (start 181.42675 116.09325) (end 181.42675 109.60325) (width 0.2) (layer "B.Cu") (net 7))
 (segment (start 177.56175 92.29075) (end 174.20425 88.93325) (width 0.2) (layer "B.Cu") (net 11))
 (segment (start 177.56175 101.10825) (end 177.56175 92.29075) (width 0.2) (layer "B.Cu") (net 11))
 (segment (start 141.1015 101.95675) (end 145.073 101.95675) (width 0.2) (layer "B.Cu") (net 21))
 (segment (start 133.9605 94.81575) (end 141.1015 101.95675) (width 0.2) (layer "B.Cu") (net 21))
 (segment (start 141.1015 99.41675) (end 145.073 99.41675) (width 0.2) (layer "B.Cu") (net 20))
 (segment (start 133.9605 92.27575) (end 141.1015 99.41675) (width 0.2) (layer "B.Cu") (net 20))
 (segment (start 179.31075 121.50925) (end 162.26275 121.50925) (width 0.2) (layer "B.Cu") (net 19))
 (segment (start 145.51331 103.01975) (end 146.136 102.39706) (width 0.2) (layer "B.Cu") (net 19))
 (segment (start 142.36175 120.60825) (end 141.46075 121.50925) (width 0.2) (layer "B.Cu") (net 19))
 (segment (start 141.46075 121.50925) (end 124.41275 121.50925) (width 0.2) (layer "B.Cu") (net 19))
 (segment (start 162.26275 121.50925) (end 161.36175 120.60825) (width 0.2) (layer "B.Cu") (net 19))
 (segment (start 146.136 97.93975) (end 145.073 96.87675) (width 0.2) (layer "B.Cu") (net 19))
 (segment (start 180.21175 120.60825) (end 179.31075 121.50925) (width 0.2) (layer "B.Cu") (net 19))
 (segment (start 186.0305 106.277) (end 180.86175 101.10825) (width 0.2) (layer "B.Cu") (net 19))
 (segment (start 124.41275 121.50925) (end 123.51175 120.60825) (width 0.2) (layer "B.Cu") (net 19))
 (segment (start 143.26275 121.50925) (end 142.36175 120.60825) (width 0.2) (layer "B.Cu") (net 19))
 (segment (start 160.46075 121.50925) (end 143.26275 121.50925) (width 0.2) (layer "B.Cu") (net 19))
 (segment (start 186.0305 114.7895) (end 186.0305 106.277) (width 0.2) (layer "B.Cu") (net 19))
 (segment (start 161.36175 120.60825) (end 160.46075 121.50925) (width 0.2) (layer "B.Cu") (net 19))
 (segment (start 123.51175 120.60825) (end 141.10025 103.01975) (width 0.2) (layer "B.Cu") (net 19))
 (segment (start 146.136 102.39706) (end 146.136 97.93975) (width 0.2) (layer "B.Cu") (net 19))
 (segment (start 141.10025 103.01975) (end 145.51331 103.01975) (width 0.2) (layer "B.Cu") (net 19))
 (segment (start 180.21175 120.60825) (end 186.0305 114.7895) (width 0.2) (layer "B.Cu") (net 19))
 (segment (start 173.8413 95.10825) (end 173.2672 95.10825) (width 0.2) (layer "F.Cu") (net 6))
 (segment (start 173.2672 95.10825) (end 172.35425 94.1953) (width 0.2) (layer "F.Cu") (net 6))
 (segment (start 167.43025 104.49675) (end 161.148 104.49675) (width 0.2) (layer "F.Cu") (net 6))
 (segment (start 175.07675 112.14325) (end 175.07675 96.3437) (width 0.2) (layer "F.Cu") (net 6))
 (segment (start 175.07675 112.14325) (end 167.43025 104.49675) (width 0.2) (layer "F.Cu") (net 6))
 (segment (start 175.07675 96.3437) (end 173.8413 95.10825) (width 0.2) (layer "F.Cu") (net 6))
 (segment (start 172.35425 94.1953) (end 172.35425 88.93325) (width 0.2) (layer "F.Cu") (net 6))
 (segment (start 152.23315 103.01975) (end 158.37615 96.87675) (width 0.2) (layer "F.Cu") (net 15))
 (segment (start 117.92675 112.14325) (end 127.05025 103.01975) (width 0.2) (layer "F.Cu") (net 15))
 (segment (start 158.37615 96.87675) (end 160.313 96.87675) (width 0.2) (layer "F.Cu") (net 15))
 (segment (start 127.05025 103.01975) (end 152.23315 103.01975) (width 0.2) (layer "F.Cu") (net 15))
 (segment (start 136.97675 112.14325) (end 143.67675 112.14325) (width 0.2) (layer "F.Cu") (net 22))
 (segment (start 156.40325 99.41675) (end 160.313 99.41675) (width 0.2) (layer "F.Cu") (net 22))
 (segment (start 143.67675 112.14325) (end 156.40325 99.41675) (width 0.2) (layer "F.Cu") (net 22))
 (segment (start 156.02675 106.243) (end 160.313 101.95675) (width 0.2) (layer "F.Cu") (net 17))
 (segment (start 156.02675 112.14325) (end 156.02675 106.243) (width 0.2) (layer "F.Cu") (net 17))
 (segment (start 173.64325 90.22225) (end 174.0353 90.22225) (width 0.2) (layer "B.Cu") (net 10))
 (segment (start 174.68025 90.8672) (end 174.68025 94.3193) (width 0.2) (layer "B.Cu") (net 10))
 (segment (start 164.6667 103.42075) (end 146.149 103.42075) (width 0.2) (layer "B.Cu") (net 10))
 (segment (start 173.1232 94.96425) (end 164.6667 103.42075) (width 0.2) (layer "B.Cu") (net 10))
 (segment (start 146.149 103.42075) (end 145.073 104.49675) (width 0.2) (layer "B.Cu") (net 10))
 (segment (start 174.0353 94.96425) (end 173.1232 94.96425) (width 0.2) (layer "B.Cu") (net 10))
 (segment (start 174.68025 94.3193) (end 174.0353 94.96425) (width 0.2) (layer "B.Cu") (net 10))
 (segment (start 172.35425 88.93325) (end 173.64325 90.22225) (width 0.2) (layer "B.Cu") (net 10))
 (segment (start 174.0353 90.22225) (end 174.68025 90.8672) (width 0.2) (layer "B.Cu") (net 10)))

